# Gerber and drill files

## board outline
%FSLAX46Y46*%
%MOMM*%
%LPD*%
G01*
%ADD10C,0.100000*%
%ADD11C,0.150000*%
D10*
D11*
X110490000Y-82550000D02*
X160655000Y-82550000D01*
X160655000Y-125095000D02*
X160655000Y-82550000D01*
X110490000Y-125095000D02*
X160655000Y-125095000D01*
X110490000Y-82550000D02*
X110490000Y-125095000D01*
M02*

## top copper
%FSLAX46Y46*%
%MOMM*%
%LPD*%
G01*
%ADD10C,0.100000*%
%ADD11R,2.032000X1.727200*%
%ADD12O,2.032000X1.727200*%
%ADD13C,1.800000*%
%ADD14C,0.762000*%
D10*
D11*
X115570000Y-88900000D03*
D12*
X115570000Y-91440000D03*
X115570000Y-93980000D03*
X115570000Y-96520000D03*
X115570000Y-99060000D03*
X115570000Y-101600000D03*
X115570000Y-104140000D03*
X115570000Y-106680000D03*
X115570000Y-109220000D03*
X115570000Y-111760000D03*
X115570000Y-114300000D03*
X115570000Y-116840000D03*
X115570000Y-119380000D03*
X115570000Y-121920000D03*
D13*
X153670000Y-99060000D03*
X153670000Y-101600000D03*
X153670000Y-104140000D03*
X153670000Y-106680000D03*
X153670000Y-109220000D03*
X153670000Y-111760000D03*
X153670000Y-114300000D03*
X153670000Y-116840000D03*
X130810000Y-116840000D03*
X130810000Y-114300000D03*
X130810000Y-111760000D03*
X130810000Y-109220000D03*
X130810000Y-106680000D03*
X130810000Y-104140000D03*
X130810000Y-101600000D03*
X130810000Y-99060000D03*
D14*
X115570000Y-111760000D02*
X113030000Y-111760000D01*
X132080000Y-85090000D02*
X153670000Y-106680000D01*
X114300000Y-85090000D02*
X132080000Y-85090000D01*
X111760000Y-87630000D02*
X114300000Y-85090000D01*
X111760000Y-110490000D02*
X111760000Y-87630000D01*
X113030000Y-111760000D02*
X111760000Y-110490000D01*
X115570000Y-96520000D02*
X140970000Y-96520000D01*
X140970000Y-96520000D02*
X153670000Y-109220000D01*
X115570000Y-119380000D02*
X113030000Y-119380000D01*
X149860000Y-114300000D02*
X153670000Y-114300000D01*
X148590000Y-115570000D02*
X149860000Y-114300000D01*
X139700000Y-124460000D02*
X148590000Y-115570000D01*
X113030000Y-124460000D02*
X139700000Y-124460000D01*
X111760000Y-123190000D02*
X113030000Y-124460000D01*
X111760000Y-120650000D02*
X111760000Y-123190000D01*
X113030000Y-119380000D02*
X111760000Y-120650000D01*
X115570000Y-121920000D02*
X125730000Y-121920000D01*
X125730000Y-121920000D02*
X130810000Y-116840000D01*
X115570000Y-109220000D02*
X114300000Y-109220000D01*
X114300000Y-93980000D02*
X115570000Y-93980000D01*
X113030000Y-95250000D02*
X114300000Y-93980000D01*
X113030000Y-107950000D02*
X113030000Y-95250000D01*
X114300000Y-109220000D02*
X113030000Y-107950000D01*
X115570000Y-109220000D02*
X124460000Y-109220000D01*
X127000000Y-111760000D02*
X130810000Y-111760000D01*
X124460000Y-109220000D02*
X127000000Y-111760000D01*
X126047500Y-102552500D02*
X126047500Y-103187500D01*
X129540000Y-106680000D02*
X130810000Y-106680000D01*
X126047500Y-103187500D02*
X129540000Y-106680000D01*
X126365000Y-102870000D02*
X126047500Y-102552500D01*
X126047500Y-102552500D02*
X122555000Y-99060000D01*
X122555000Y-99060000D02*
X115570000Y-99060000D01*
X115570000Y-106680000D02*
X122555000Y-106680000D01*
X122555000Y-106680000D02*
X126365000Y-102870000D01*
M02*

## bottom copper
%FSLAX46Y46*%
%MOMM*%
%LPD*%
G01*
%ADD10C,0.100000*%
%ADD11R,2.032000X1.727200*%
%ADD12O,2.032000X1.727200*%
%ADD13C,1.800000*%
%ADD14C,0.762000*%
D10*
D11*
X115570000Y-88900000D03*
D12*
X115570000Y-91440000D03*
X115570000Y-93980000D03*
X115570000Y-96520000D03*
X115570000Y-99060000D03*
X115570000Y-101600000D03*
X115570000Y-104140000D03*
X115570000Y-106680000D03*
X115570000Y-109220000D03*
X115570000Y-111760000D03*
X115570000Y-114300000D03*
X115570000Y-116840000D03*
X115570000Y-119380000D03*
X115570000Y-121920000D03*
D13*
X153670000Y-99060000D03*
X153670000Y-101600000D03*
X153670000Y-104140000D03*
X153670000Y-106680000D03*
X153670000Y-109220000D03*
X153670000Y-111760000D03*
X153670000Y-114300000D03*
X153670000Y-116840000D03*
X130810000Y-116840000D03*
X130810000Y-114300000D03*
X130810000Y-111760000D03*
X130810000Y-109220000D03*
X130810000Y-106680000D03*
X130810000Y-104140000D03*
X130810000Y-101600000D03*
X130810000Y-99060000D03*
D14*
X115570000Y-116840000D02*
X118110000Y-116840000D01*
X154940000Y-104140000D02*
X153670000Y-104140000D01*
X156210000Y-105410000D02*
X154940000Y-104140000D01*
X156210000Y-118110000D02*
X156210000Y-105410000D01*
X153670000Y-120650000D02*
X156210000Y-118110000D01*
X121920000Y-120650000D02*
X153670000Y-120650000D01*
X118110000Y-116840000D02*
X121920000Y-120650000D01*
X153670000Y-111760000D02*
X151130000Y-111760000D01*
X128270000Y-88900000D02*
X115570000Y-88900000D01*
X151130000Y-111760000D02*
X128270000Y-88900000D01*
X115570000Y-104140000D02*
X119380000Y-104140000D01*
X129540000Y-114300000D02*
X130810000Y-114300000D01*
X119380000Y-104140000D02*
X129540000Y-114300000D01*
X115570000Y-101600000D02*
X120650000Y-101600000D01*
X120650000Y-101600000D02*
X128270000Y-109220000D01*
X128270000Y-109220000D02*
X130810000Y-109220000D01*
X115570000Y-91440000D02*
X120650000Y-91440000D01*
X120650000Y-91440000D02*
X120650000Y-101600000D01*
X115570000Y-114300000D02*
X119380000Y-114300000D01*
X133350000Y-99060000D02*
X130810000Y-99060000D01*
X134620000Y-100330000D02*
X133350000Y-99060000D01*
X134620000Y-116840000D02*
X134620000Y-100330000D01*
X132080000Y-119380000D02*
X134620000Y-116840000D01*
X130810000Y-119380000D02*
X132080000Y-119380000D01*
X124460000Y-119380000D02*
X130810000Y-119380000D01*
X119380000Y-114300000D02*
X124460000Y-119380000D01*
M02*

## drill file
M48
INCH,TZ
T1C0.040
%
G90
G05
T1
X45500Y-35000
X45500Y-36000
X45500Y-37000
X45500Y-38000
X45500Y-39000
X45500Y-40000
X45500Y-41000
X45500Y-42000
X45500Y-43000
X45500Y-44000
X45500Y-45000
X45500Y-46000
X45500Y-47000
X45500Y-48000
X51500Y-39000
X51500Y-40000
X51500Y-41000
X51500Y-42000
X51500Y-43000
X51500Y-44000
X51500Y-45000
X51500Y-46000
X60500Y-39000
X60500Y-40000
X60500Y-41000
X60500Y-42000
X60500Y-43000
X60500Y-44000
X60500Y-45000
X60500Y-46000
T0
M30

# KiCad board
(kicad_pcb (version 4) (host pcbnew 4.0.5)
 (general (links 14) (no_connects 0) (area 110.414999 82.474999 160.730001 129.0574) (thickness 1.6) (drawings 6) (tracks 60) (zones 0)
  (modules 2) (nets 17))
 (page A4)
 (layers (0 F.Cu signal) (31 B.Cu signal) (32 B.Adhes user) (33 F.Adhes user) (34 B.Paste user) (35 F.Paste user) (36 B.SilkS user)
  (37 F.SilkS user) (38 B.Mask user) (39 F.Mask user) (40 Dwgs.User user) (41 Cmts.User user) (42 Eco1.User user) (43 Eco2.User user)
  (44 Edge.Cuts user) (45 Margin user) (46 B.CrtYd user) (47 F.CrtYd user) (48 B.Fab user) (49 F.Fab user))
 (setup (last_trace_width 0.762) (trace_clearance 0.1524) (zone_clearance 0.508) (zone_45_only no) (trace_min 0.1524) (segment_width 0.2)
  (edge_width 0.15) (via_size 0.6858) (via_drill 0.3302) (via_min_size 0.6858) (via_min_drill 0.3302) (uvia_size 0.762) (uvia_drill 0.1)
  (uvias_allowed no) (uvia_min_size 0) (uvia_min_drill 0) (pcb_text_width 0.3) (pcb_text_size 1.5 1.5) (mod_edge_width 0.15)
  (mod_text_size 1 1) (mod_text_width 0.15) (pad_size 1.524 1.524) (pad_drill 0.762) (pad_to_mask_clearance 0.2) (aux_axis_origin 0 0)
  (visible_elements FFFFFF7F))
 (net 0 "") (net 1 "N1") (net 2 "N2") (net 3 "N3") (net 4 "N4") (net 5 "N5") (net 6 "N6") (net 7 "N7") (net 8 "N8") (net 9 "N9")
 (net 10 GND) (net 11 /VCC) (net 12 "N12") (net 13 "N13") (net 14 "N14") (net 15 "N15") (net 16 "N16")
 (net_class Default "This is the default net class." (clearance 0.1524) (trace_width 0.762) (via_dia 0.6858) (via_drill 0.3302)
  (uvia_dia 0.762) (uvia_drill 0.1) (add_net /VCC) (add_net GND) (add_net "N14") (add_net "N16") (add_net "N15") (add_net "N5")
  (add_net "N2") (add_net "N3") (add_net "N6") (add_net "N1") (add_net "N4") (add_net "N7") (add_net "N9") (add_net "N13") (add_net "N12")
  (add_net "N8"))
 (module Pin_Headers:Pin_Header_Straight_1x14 (layer F.Cu) (at 115.57 88.9)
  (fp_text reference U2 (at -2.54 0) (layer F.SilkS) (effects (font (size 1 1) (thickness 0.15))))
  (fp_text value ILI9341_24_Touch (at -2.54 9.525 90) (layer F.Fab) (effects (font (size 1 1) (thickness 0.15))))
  (pad 1 thru_hole rect (at 0 0) (size 2.032 1.7272) (drill 1.016) (layers *.Cu *.Mask) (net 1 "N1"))
  (pad 2 thru_hole oval (at 0 2.54) (size 2.032 1.7272) (drill 1.016) (layers *.Cu *.Mask) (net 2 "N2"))
  (pad 3 thru_hole oval (at 0 5.08) (size 2.032 1.7272) (drill 1.016) (layers *.Cu *.Mask) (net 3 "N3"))
  (pad 4 thru_hole oval (at 0 7.62) (size 2.032 1.7272) (drill 1.016) (layers *.Cu *.Mask) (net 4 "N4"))
  (pad 5 thru_hole oval (at 0 10.16) (size 2.032 1.7272) (drill 1.016) (layers *.Cu *.Mask) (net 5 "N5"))
  (pad 6 thru_hole oval (at 0 12.7) (size 2.032 1.7272) (drill 1.016) (layers *.Cu *.Mask) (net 2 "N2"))
  (pad 7 thru_hole oval (at 0 15.24) (size 2.032 1.7272) (drill 1.016) (layers *.Cu *.Mask) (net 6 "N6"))
  (pad 8 thru_hole oval (at 0 17.78) (size 2.032 1.7272) (drill 1.016) (layers *.Cu *.Mask) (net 5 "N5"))
  (pad 9 thru_hole oval (at 0 20.32) (size 2.032 1.7272) (drill 1.016) (layers *.Cu *.Mask) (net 3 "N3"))
  (pad 10 thru_hole oval (at 0 22.86) (size 2.032 1.7272) (drill 1.016) (layers *.Cu *.Mask) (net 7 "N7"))
  (pad 11 thru_hole oval (at 0 25.4) (size 2.032 1.7272) (drill 1.016) (layers *.Cu *.Mask) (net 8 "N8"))
  (pad 12 thru_hole oval (at 0 27.94) (size 2.032 1.7272) (drill 1.016) (layers *.Cu *.Mask) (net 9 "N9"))
  (pad 13 thru_hole oval (at 0 30.48) (size 2.032 1.7272) (drill 1.016) (layers *.Cu *.Mask) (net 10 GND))
  (pad 14 thru_hole oval (at 0 33.02) (size 2.032 1.7272) (drill 1.016) (layers *.Cu *.Mask) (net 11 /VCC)))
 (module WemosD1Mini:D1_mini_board (layer B.Cu) (at 142.24 109.22 180)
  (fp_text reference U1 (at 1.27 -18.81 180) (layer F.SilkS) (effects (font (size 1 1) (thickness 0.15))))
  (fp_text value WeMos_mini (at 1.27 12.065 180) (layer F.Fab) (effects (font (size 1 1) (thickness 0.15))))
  (pad 8 thru_hole circle (at -11.43 10.16 180) (size 1.8 1.8) (drill 1.016) (layers *.Cu *.Mask B.SilkS) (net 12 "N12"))
  (pad 7 thru_hole circle (at -11.43 7.62 180) (size 1.8 1.8) (drill 1.016) (layers *.Cu *.Mask B.SilkS) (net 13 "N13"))
  (pad 6 thru_hole circle (at -11.43 5.08 180) (size 1.8 1.8) (drill 1.016) (layers *.Cu *.Mask B.SilkS) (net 9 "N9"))
  (pad 5 thru_hole circle (at -11.43 2.54 180) (size 1.8 1.8) (drill 1.016) (layers *.Cu *.Mask B.SilkS) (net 7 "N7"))
  (pad 4 thru_hole circle (at -11.43 0 180) (size 1.8 1.8) (drill 1.016) (layers *.Cu *.Mask B.SilkS) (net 4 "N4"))
  (pad 3 thru_hole circle (at -11.43 -2.54 180) (size 1.8 1.8) (drill 1.016) (layers *.Cu *.Mask B.SilkS) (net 1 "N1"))
  (pad 2 thru_hole circle (at -11.43 -5.08 180) (size 1.8 1.8) (drill 1.016) (layers *.Cu *.Mask B.SilkS) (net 10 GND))
  (pad 1 thru_hole circle (at -11.43 -7.62 180) (size 1.8 1.8) (drill 1.016) (layers *.Cu *.Mask B.SilkS) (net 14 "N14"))
  (pad 16 thru_hole circle (at 11.43 -7.62 180) (size 1.8 1.8) (drill 1.016) (layers *.Cu *.Mask B.SilkS) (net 11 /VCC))
  (pad 15 thru_hole circle (at 11.43 -5.08 180) (size 1.8 1.8) (drill 1.016) (layers *.Cu *.Mask B.SilkS) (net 6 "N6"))
  (pad 14 thru_hole circle (at 11.43 -2.54 180) (size 1.8 1.8) (drill 1.016) (layers *.Cu *.Mask B.SilkS) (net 3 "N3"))
  (pad 13 thru_hole circle (at 11.43 0 180) (size 1.8 1.8) (drill 1.016) (layers *.Cu *.Mask B.SilkS) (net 2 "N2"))
  (pad 12 thru_hole circle (at 11.43 2.54 180) (size 1.8 1.8) (drill 1.016) (layers *.Cu *.Mask B.SilkS) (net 5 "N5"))
  (pad 11 thru_hole circle (at 11.43 5.08 180) (size 1.8 1.8) (drill 1.016) (layers *.Cu *.Mask B.SilkS) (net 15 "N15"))
  (pad 10 thru_hole circle (at 11.43 7.62 180) (size 1.8 1.8) (drill 1.016) (layers *.Cu *.Mask B.SilkS) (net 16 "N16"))
  (pad 9 thru_hole circle (at 11.43 10.16 180) (size 1.8 1.8) (drill 1.016) (layers *.Cu *.Mask B.SilkS) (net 8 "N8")))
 (gr_line (start 110.49 82.55) (end 160.655 82.55) (angle 90) (layer Edge.Cuts) (width 0.15))
 (gr_line (start 160.655 125.095) (end 160.655 82.55) (angle 90) (layer Edge.Cuts) (width 0.15))
 (gr_line (start 110.49 125.095) (end 160.655 125.095) (angle 90) (layer Edge.Cuts) (width 0.15))
 (gr_line (start 110.49 82.55) (end 110.49 125.095) (angle 90) (layer Edge.Cuts) (width 0.15))
 (segment (start 115.57 116.84) (end 118.11 116.84) (width 0.762) (layer B.Cu) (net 9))
 (segment (start 154.94 104.14) (end 153.67 104.14) (width 0.762) (layer B.Cu) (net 9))
 (segment (start 156.21 105.41) (end 154.94 104.14) (width 0.762) (layer B.Cu) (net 9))
 (segment (start 156.21 118.11) (end 156.21 105.41) (width 0.762) (layer B.Cu) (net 9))
 (segment (start 153.67 120.65) (end 156.21 118.11) (width 0.762) (layer B.Cu) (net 9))
 (segment (start 121.92 120.65) (end 153.67 120.65) (width 0.762) (layer B.Cu) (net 9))
 (segment (start 118.11 116.84) (end 121.92 120.65) (width 0.762) (layer B.Cu) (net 9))
 (segment (start 115.57 111.76) (end 113.03 111.76) (width 0.762) (layer F.Cu) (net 7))
 (segment (start 132.08 85.09) (end 153.67 106.68) (width 0.762) (layer F.Cu) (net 7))
 (segment (start 114.3 85.09) (end 132.08 85.09) (width 0.762) (layer F.Cu) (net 7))
 (segment (start 111.76 87.63) (end 114.3 85.09) (width 0.762) (layer F.Cu) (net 7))
 (segment (start 111.76 110.49) (end 111.76 87.63) (width 0.762) (layer F.Cu) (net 7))
 (segment (start 113.03 111.76) (end 111.76 110.49) (width 0.762) (layer F.Cu) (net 7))
 (segment (start 115.57 96.52) (end 140.97 96.52) (width 0.762) (layer F.Cu) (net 4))
 (segment (start 140.97 96.52) (end 153.67 109.22) (width 0.762) (layer F.Cu) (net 4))
 (segment (start 153.67 111.76) (end 151.13 111.76) (width 0.762) (layer B.Cu) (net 1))
 (segment (start 128.27 88.9) (end 115.57 88.9) (width 0.762) (layer B.Cu) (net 1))
 (segment (start 151.13 111.76) (end 128.27 88.9) (width 0.762) (layer B.Cu) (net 1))
 (segment (start 115.57 119.38) (end 113.03 119.38) (width 0.762) (layer F.Cu) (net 10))
 (segment (start 149.86 114.3) (end 153.67 114.3) (width 0.762) (layer F.Cu) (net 10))
 (segment (start 148.59 115.57) (end 149.86 114.3) (width 0.762) (layer F.Cu) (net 10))
 (segment (start 139.7 124.46) (end 148.59 115.57) (width 0.762) (layer F.Cu) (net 10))
 (segment (start 113.03 124.46) (end 139.7 124.46) (width 0.762) (layer F.Cu) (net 10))
 (segment (start 111.76 123.19) (end 113.03 124.46) (width 0.762) (layer F.Cu) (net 10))
 (segment (start 111.76 120.65) (end 111.76 123.19) (width 0.762) (layer F.Cu) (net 10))
 (segment (start 113.03 119.38) (end 111.76 120.65) (width 0.762) (layer F.Cu) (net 10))
 (segment (start 115.57 121.92) (end 125.73 121.92) (width 0.762) (layer F.Cu) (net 11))
 (segment (start 125.73 121.92) (end 130.81 116.84) (width 0.762) (layer F.Cu) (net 11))
 (segment (start 115.57 104.14) (end 119.38 104.14) (width 0.762) (layer B.Cu) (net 6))
 (segment (start 129.54 114.3) (end 130.81 114.3) (width 0.762) (layer B.Cu) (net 6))
 (segment (start 119.38 104.14) (end 129.54 114.3) (width 0.762) (layer B.Cu) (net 6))
 (segment (start 115.57 109.22) (end 114.3 109.22) (width 0.762) (layer F.Cu) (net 3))
 (segment (start 114.3 93.98) (end 115.57 93.98) (width 0.762) (layer F.Cu) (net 3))
 (segment (start 113.03 95.25) (end 114.3 93.98) (width 0.762) (layer F.Cu) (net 3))
 (segment (start 113.03 107.95) (end 113.03 95.25) (width 0.762) (layer F.Cu) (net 3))
 (segment (start 114.3 109.22) (end 113.03 107.95) (width 0.762) (layer F.Cu) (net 3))
 (segment (start 115.57 109.22) (end 124.46 109.22) (width 0.762) (layer F.Cu) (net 3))
 (segment (start 127 111.76) (end 130.81 111.76) (width 0.762) (layer F.Cu) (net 3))
 (segment (start 124.46 109.22) (end 127 111.76) (width 0.762) (layer F.Cu) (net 3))
 (segment (start 115.57 101.6) (end 120.65 101.6) (width 0.762) (layer B.Cu) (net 2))
 (segment (start 120.65 101.6) (end 128.27 109.22) (width 0.762) (layer B.Cu) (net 2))
 (segment (start 128.27 109.22) (end 130.81 109.22) (width 0.762) (layer B.Cu) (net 2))
 (segment (start 115.57 91.44) (end 120.65 91.44) (width 0.762) (layer B.Cu) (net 2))
 (segment (start 120.65 91.44) (end 120.65 101.6) (width 0.762) (layer B.Cu) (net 2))
 (segment (start 126.0475 102.5525) (end 126.0475 103.1875) (width 0.762) (layer F.Cu) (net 5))
 (segment (start 129.54 106.68) (end 130.81 106.68) (width 0.762) (layer F.Cu) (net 5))
 (segment (start 126.0475 103.1875) (end 129.54 106.68) (width 0.762) (layer F.Cu) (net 5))
 (segment (start 126.365 102.87) (end 126.0475 102.5525) (width 0.762) (layer F.Cu) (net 5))
 (segment (start 126.0475 102.5525) (end 122.555 99.06) (width 0.762) (layer F.Cu) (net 5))
 (segment (start 122.555 99.06) (end 115.57 99.06) (width 0.762) (layer F.Cu) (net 5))
 (segment (start 115.57 106.68) (end 122.555 106.68) (width 0.762) (layer F.Cu) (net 5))
 (segment (start 122.555 106.68) (end 126.365 102.87) (width 0.762) (layer F.Cu) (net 5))
 (segment (start 115.57 114.3) (end 119.38 114.3) (width 0.762) (layer B.Cu) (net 8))
 (segment (start 133.35 99.06) (end 130.81 99.06) (width 0.762) (layer B.Cu) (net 8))
 (segment (start 134.62 100.33) (end 133.35 99.06) (width 0.762) (layer B.Cu) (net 8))
 (segment (start 134.62 116.84) (end 134.62 100.33) (width 0.762) (layer B.Cu) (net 8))
 (segment (start 132.08 119.38) (end 134.62 116.84) (width 0.762) (layer B.Cu) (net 8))
 (segment (start 130.81 119.38) (end 132.08 119.38) (width 0.762) (layer B.Cu) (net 8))
 (segment (start 124.46 119.38) (end 130.81 119.38) (width 0.762) (layer B.Cu) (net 8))
 (segment (start 119.38 114.3) (end 124.46 119.38) (width 0.762) (layer B.Cu) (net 8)))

